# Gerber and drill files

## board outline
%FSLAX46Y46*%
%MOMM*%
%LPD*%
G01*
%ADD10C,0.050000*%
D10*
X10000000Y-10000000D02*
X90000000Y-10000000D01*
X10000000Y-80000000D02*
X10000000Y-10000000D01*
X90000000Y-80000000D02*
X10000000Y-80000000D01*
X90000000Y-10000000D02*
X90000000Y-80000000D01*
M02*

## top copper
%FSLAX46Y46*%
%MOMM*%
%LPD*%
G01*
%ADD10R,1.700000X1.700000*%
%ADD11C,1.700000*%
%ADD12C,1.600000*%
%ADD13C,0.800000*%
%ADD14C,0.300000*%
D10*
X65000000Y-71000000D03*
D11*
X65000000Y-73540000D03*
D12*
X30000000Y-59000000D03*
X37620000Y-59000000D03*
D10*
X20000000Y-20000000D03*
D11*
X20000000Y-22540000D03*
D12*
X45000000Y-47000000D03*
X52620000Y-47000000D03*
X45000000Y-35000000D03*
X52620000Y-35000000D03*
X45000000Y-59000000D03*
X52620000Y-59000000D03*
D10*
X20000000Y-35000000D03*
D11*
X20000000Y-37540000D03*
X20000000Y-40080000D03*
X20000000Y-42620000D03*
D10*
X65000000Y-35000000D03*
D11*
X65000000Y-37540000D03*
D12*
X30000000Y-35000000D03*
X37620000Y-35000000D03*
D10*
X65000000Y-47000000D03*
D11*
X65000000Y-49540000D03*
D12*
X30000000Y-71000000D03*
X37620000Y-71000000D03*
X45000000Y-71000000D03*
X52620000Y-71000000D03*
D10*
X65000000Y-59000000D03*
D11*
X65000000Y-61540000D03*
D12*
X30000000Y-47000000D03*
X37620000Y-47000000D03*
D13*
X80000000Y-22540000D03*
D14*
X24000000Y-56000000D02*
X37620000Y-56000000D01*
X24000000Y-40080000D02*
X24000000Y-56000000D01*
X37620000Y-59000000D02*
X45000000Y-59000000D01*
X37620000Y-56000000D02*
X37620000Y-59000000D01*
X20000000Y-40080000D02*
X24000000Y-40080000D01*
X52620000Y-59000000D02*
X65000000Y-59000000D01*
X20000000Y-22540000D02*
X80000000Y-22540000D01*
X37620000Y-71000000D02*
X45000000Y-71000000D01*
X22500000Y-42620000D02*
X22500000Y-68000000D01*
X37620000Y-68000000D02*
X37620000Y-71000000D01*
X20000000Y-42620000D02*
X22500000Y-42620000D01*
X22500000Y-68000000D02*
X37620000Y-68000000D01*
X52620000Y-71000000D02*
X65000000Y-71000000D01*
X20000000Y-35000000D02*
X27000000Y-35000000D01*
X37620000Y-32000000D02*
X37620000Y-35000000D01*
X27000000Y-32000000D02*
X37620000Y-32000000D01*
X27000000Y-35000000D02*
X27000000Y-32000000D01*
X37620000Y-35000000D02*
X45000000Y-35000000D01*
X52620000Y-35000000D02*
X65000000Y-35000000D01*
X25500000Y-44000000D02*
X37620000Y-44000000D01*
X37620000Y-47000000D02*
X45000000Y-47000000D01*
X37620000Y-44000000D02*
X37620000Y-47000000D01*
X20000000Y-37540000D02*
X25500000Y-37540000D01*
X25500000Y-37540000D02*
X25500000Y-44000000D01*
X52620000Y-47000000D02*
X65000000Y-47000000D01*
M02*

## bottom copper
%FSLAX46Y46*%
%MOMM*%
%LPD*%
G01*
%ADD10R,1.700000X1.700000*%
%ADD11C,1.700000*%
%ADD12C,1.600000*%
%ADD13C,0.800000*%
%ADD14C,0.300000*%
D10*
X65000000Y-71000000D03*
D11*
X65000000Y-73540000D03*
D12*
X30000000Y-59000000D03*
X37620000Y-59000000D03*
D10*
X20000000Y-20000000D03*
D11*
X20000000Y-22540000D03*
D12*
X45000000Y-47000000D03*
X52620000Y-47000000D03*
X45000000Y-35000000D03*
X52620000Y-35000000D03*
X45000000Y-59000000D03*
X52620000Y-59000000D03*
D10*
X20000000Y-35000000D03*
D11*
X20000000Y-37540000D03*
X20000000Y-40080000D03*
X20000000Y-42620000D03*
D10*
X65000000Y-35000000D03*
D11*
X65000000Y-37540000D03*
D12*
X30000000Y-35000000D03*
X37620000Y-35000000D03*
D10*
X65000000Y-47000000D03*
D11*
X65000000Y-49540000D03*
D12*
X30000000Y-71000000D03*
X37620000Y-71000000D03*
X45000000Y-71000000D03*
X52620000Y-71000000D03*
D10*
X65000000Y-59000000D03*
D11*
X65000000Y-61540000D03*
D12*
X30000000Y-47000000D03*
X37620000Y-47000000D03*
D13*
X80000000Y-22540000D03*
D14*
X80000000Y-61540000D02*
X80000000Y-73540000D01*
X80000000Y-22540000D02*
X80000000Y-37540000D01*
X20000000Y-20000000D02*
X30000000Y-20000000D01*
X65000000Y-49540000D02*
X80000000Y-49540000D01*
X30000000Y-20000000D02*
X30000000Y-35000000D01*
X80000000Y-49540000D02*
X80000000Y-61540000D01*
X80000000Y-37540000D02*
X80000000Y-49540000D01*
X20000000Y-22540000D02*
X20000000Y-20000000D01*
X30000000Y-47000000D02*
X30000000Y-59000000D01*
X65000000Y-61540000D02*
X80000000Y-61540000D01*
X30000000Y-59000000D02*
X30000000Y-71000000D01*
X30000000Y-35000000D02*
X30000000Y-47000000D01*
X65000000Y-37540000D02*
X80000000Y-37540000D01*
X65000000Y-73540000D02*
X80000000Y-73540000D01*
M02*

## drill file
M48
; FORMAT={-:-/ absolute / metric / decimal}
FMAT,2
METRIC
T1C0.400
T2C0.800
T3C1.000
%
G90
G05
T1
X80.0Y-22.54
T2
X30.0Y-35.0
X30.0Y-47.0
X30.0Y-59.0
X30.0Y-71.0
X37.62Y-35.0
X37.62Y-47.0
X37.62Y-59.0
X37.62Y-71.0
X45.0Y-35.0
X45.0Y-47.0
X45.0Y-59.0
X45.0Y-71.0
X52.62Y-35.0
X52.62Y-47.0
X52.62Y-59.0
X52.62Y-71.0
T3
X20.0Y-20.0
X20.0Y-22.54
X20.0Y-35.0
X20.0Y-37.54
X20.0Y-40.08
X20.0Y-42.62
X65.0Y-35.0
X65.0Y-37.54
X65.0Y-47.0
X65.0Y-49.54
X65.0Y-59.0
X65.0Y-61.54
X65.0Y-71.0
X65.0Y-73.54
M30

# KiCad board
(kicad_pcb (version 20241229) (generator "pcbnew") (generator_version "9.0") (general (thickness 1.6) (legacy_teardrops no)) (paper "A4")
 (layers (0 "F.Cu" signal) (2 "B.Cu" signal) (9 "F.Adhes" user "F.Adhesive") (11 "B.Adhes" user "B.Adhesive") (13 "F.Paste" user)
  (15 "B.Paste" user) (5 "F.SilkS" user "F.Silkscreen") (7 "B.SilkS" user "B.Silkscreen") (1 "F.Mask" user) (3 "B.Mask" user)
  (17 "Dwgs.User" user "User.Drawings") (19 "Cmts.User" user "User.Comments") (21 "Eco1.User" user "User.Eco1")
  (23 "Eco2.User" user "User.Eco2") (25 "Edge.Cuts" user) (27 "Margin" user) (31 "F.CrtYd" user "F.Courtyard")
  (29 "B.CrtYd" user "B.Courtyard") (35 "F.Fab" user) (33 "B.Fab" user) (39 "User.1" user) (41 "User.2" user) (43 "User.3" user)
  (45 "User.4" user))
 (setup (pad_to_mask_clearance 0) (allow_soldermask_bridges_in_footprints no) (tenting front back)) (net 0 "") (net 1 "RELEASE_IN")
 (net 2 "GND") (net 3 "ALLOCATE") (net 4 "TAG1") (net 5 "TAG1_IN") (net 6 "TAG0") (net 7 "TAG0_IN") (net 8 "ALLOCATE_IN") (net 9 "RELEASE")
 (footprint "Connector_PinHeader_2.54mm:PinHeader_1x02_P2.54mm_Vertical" (layer "F.Cu") (at 65 71)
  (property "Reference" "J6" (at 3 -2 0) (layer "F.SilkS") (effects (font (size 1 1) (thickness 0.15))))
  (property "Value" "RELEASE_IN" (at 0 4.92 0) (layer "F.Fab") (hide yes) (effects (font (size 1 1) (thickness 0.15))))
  (pad "1" thru_hole rect (at 0 0) (size 1.7 1.7) (drill 1) (layers "*.Cu" "*.Mask") (remove_unused_layers no) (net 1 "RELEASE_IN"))
  (pad "2" thru_hole circle (at 0 2.54) (size 1.7 1.7) (drill 1) (layers "*.Cu" "*.Mask") (remove_unused_layers no) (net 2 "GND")))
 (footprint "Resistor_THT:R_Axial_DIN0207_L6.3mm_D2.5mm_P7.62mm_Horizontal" (layer "F.Cu") (at 30 59)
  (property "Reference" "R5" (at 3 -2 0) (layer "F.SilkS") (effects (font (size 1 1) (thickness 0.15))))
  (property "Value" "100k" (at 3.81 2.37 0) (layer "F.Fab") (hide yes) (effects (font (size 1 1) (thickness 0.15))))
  (pad "1" thru_hole circle (at 0 0) (size 1.6 1.6) (drill 0.8) (layers "*.Cu" "*.Mask") (remove_unused_layers no) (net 2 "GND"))
  (pad "2" thru_hole circle (at 7.62 0) (size 1.6 1.6) (drill 0.8) (layers "*.Cu" "*.Mask") (remove_unused_layers no) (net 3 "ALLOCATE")))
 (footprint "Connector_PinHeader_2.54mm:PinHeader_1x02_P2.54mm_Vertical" (layer "F.Cu") (at 20 20)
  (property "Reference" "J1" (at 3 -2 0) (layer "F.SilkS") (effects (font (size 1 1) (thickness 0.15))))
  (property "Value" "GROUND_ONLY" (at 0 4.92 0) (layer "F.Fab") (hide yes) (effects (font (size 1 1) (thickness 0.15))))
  (pad "1" thru_hole rect (at 0 0) (size 1.7 1.7) (drill 1) (layers "*.Cu" "*.Mask") (remove_unused_layers no) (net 2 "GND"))
  (pad "2" thru_hole circle (at 0 2.54) (size 1.7 1.7) (drill 1) (layers "*.Cu" "*.Mask") (remove_unused_layers no) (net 2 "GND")))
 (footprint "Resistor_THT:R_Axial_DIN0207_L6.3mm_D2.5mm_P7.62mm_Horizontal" (layer "F.Cu") (at 45 47)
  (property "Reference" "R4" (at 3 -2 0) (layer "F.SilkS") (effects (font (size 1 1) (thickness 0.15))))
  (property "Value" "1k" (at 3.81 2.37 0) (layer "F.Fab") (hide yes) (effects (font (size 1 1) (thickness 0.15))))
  (pad "1" thru_hole circle (at 0 0) (size 1.6 1.6) (drill 0.8) (layers "*.Cu" "*.Mask") (remove_unused_layers no) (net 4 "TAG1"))
  (pad "2" thru_hole circle (at 7.62 0) (size 1.6 1.6) (drill 0.8) (layers "*.Cu" "*.Mask") (remove_unused_layers no) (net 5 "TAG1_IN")))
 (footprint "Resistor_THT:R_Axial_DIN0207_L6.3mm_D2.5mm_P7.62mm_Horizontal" (layer "F.Cu") (at 45 35)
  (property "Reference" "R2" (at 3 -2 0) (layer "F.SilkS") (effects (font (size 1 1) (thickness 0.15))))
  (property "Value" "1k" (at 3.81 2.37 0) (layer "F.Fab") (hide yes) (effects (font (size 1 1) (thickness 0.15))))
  (pad "1" thru_hole circle (at 0 0) (size 1.6 1.6) (drill 0.8) (layers "*.Cu" "*.Mask") (remove_unused_layers no) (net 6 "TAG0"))
  (pad "2" thru_hole circle (at 7.62 0) (size 1.6 1.6) (drill 0.8) (layers "*.Cu" "*.Mask") (remove_unused_layers no) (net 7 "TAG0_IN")))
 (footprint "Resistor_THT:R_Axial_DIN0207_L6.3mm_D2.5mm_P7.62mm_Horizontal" (layer "F.Cu") (at 45 59)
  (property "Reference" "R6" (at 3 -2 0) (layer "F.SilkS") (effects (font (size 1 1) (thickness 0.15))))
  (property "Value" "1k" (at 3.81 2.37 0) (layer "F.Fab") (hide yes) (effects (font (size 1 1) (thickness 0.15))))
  (pad "1" thru_hole circle (at 0 0) (size 1.6 1.6) (drill 0.8) (layers "*.Cu" "*.Mask") (remove_unused_layers no) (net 3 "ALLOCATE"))
  (pad "2" thru_hole circle (at 7.62 0) (size 1.6 1.6) (drill 0.8) (layers "*.Cu" "*.Mask") (remove_unused_layers no) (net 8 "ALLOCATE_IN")))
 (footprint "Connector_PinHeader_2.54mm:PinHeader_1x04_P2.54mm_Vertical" (layer "F.Cu") (at 20 35)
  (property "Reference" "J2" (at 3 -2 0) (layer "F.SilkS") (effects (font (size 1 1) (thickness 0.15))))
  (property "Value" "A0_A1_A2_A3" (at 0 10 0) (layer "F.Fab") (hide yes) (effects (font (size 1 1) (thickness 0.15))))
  (pad "1" thru_hole rect (at 0 0) (size 1.7 1.7) (drill 1) (layers "*.Cu" "*.Mask") (remove_unused_layers no) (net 6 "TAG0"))
  (pad "2" thru_hole circle (at 0 2.54) (size 1.7 1.7) (drill 1) (layers "*.Cu" "*.Mask") (remove_unused_layers no) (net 4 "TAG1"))
  (pad "3" thru_hole circle (at 0 5.08) (size 1.7 1.7) (drill 1) (layers "*.Cu" "*.Mask") (remove_unused_layers no) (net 3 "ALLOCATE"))
  (pad "4" thru_hole circle (at 0 7.62) (size 1.7 1.7) (drill 1) (layers "*.Cu" "*.Mask") (remove_unused_layers no) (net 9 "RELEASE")))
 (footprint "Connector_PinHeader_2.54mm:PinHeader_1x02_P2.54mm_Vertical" (layer "F.Cu") (at 65 35)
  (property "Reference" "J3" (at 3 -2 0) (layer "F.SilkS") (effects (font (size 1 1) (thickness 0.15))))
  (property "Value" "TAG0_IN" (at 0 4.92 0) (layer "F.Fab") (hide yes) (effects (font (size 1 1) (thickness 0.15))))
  (pad "1" thru_hole rect (at 0 0) (size 1.7 1.7) (drill 1) (layers "*.Cu" "*.Mask") (remove_unused_layers no) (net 7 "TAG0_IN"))
  (pad "2" thru_hole circle (at 0 2.54) (size 1.7 1.7) (drill 1) (layers "*.Cu" "*.Mask") (remove_unused_layers no) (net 2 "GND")))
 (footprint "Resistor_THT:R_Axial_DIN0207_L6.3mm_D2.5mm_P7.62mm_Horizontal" (layer "F.Cu") (at 30 35)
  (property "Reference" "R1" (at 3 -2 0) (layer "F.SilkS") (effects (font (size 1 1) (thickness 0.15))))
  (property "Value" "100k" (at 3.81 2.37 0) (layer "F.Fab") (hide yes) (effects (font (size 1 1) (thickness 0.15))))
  (pad "1" thru_hole circle (at 0 0) (size 1.6 1.6) (drill 0.8) (layers "*.Cu" "*.Mask") (remove_unused_layers no) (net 2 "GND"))
  (pad "2" thru_hole circle (at 7.62 0) (size 1.6 1.6) (drill 0.8) (layers "*.Cu" "*.Mask") (remove_unused_layers no) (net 6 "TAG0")))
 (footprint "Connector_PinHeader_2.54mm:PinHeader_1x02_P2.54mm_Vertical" (layer "F.Cu") (at 65 47)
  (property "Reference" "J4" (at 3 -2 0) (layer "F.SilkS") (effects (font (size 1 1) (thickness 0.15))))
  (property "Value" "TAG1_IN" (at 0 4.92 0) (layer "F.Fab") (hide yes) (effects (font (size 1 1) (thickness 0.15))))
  (pad "1" thru_hole rect (at 0 0) (size 1.7 1.7) (drill 1) (layers "*.Cu" "*.Mask") (remove_unused_layers no) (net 5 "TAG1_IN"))
  (pad "2" thru_hole circle (at 0 2.54) (size 1.7 1.7) (drill 1) (layers "*.Cu" "*.Mask") (remove_unused_layers no) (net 2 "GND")))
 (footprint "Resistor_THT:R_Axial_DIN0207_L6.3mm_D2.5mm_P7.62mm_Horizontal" (layer "F.Cu") (at 30 71)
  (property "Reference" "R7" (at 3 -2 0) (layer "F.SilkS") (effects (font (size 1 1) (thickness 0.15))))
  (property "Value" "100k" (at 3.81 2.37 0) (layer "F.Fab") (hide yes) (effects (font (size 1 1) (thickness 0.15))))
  (pad "1" thru_hole circle (at 0 0) (size 1.6 1.6) (drill 0.8) (layers "*.Cu" "*.Mask") (remove_unused_layers no) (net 2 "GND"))
  (pad "2" thru_hole circle (at 7.62 0) (size 1.6 1.6) (drill 0.8) (layers "*.Cu" "*.Mask") (remove_unused_layers no) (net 9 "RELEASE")))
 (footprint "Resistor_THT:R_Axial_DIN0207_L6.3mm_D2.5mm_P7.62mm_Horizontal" (layer "F.Cu") (at 45 71)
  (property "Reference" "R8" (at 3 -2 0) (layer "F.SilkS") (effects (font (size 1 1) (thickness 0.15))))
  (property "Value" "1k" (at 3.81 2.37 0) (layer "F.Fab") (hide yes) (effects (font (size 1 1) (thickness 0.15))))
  (pad "1" thru_hole circle (at 0 0) (size 1.6 1.6) (drill 0.8) (layers "*.Cu" "*.Mask") (remove_unused_layers no) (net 9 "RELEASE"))
  (pad "2" thru_hole circle (at 7.62 0) (size 1.6 1.6) (drill 0.8) (layers "*.Cu" "*.Mask") (remove_unused_layers no) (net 1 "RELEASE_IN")))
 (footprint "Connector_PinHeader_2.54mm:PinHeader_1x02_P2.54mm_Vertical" (layer "F.Cu") (at 65 59)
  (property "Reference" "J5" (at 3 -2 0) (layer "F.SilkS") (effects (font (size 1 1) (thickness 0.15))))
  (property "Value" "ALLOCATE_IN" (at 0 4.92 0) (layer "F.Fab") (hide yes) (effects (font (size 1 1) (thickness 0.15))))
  (pad "1" thru_hole rect (at 0 0) (size 1.7 1.7) (drill 1) (layers "*.Cu" "*.Mask") (remove_unused_layers no) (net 8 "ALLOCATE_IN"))
  (pad "2" thru_hole circle (at 0 2.54) (size 1.7 1.7) (drill 1) (layers "*.Cu" "*.Mask") (remove_unused_layers no) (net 2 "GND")))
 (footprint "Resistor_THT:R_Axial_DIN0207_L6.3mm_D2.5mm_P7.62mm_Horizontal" (layer "F.Cu") (at 30 47)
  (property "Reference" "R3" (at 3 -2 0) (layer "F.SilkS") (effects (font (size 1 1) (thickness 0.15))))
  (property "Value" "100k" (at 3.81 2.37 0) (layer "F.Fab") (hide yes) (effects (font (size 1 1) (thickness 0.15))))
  (pad "1" thru_hole circle (at 0 0) (size 1.6 1.6) (drill 0.8) (layers "*.Cu" "*.Mask") (remove_unused_layers no) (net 2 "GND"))
  (pad "2" thru_hole circle (at 7.62 0) (size 1.6 1.6) (drill 0.8) (layers "*.Cu" "*.Mask") (remove_unused_layers no) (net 4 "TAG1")))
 (gr_line (start 10 10) (end 90 10) (stroke (width 0.05) (type default)) (layer "Edge.Cuts"))
 (gr_line (start 10 80) (end 10 10) (stroke (width 0.05) (type default)) (layer "Edge.Cuts"))
 (gr_line (start 90 80) (end 10 80) (stroke (width 0.05) (type default)) (layer "Edge.Cuts"))
 (gr_line (start 90 10) (end 90 80) (stroke (width 0.05) (type default)) (layer "Edge.Cuts"))
 (segment (start 24 56) (end 37.62 56) (width 0.3) (layer "F.Cu") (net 3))
 (segment (start 24 40.08) (end 24 56) (width 0.3) (layer "F.Cu") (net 3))
 (segment (start 37.62 59) (end 45 59) (width 0.3) (layer "F.Cu") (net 3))
 (segment (start 37.62 56) (end 37.62 59) (width 0.3) (layer "F.Cu") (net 3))
 (segment (start 20 40.08) (end 24 40.08) (width 0.3) (layer "F.Cu") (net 3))
 (segment (start 52.62 59) (end 65 59) (width 0.3) (layer "F.Cu") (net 8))
 (segment (start 20 22.54) (end 80 22.54) (width 0.3) (layer "F.Cu") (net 2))
 (via (at 80 22.54) (size 0.8) (drill 0.4) (layers "F.Cu" "B.Cu") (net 2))
 (segment (start 80 61.54) (end 80 73.54) (width 0.3) (layer "B.Cu") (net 2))
 (segment (start 80 22.54) (end 80 37.54) (width 0.3) (layer "B.Cu") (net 2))
 (segment (start 20 20) (end 30 20) (width 0.3) (layer "B.Cu") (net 2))
 (segment (start 65 49.54) (end 80 49.54) (width 0.3) (layer "B.Cu") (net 2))
 (segment (start 30 20) (end 30 35) (width 0.3) (layer "B.Cu") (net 2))
 (segment (start 80 49.54) (end 80 61.54) (width 0.3) (layer "B.Cu") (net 2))
 (segment (start 80 37.54) (end 80 49.54) (width 0.3) (layer "B.Cu") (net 2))
 (segment (start 20 22.54) (end 20 20) (width 0.3) (layer "B.Cu") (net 2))
 (segment (start 30 47) (end 30 59) (width 0.3) (layer "B.Cu") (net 2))
 (segment (start 65 61.54) (end 80 61.54) (width 0.3) (layer "B.Cu") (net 2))
 (segment (start 30 59) (end 30 71) (width 0.3) (layer "B.Cu") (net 2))
 (segment (start 30 35) (end 30 47) (width 0.3) (layer "B.Cu") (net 2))
 (segment (start 65 37.54) (end 80 37.54) (width 0.3) (layer "B.Cu") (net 2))
 (segment (start 65 73.54) (end 80 73.54) (width 0.3) (layer "B.Cu") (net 2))
 (segment (start 37.62 71) (end 45 71) (width 0.3) (layer "F.Cu") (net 9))
 (segment (start 22.5 42.62) (end 22.5 68) (width 0.3) (layer "F.Cu") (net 9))
 (segment (start 37.62 68) (end 37.62 71) (width 0.3) (layer "F.Cu") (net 9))
 (segment (start 20 42.62) (end 22.5 42.62) (width 0.3) (layer "F.Cu") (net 9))
 (segment (start 22.5 68) (end 37.62 68) (width 0.3) (layer "F.Cu") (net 9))
 (segment (start 52.62 71) (end 65 71) (width 0.3) (layer "F.Cu") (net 1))
 (segment (start 20 35) (end 27 35) (width 0.3) (layer "F.Cu") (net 6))
 (segment (start 37.62 32) (end 37.62 35) (width 0.3) (layer "F.Cu") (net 6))
 (segment (start 27 32) (end 37.62 32) (width 0.3) (layer "F.Cu") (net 6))
 (segment (start 27 35) (end 27 32) (width 0.3) (layer "F.Cu") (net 6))
 (segment (start 37.62 35) (end 45 35) (width 0.3) (layer "F.Cu") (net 6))
 (segment (start 52.62 35) (end 65 35) (width 0.3) (layer "F.Cu") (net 7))
 (segment (start 25.5 44) (end 37.62 44) (width 0.3) (layer "F.Cu") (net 4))
 (segment (start 37.62 47) (end 45 47) (width 0.3) (layer "F.Cu") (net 4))
 (segment (start 37.62 44) (end 37.62 47) (width 0.3) (layer "F.Cu") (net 4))
 (segment (start 20 37.54) (end 25.5 37.54) (width 0.3) (layer "F.Cu") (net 4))
 (segment (start 25.5 37.54) (end 25.5 44) (width 0.3) (layer "F.Cu") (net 4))
 (segment (start 52.62 47) (end 65 47) (width 0.3) (layer "F.Cu") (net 5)))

